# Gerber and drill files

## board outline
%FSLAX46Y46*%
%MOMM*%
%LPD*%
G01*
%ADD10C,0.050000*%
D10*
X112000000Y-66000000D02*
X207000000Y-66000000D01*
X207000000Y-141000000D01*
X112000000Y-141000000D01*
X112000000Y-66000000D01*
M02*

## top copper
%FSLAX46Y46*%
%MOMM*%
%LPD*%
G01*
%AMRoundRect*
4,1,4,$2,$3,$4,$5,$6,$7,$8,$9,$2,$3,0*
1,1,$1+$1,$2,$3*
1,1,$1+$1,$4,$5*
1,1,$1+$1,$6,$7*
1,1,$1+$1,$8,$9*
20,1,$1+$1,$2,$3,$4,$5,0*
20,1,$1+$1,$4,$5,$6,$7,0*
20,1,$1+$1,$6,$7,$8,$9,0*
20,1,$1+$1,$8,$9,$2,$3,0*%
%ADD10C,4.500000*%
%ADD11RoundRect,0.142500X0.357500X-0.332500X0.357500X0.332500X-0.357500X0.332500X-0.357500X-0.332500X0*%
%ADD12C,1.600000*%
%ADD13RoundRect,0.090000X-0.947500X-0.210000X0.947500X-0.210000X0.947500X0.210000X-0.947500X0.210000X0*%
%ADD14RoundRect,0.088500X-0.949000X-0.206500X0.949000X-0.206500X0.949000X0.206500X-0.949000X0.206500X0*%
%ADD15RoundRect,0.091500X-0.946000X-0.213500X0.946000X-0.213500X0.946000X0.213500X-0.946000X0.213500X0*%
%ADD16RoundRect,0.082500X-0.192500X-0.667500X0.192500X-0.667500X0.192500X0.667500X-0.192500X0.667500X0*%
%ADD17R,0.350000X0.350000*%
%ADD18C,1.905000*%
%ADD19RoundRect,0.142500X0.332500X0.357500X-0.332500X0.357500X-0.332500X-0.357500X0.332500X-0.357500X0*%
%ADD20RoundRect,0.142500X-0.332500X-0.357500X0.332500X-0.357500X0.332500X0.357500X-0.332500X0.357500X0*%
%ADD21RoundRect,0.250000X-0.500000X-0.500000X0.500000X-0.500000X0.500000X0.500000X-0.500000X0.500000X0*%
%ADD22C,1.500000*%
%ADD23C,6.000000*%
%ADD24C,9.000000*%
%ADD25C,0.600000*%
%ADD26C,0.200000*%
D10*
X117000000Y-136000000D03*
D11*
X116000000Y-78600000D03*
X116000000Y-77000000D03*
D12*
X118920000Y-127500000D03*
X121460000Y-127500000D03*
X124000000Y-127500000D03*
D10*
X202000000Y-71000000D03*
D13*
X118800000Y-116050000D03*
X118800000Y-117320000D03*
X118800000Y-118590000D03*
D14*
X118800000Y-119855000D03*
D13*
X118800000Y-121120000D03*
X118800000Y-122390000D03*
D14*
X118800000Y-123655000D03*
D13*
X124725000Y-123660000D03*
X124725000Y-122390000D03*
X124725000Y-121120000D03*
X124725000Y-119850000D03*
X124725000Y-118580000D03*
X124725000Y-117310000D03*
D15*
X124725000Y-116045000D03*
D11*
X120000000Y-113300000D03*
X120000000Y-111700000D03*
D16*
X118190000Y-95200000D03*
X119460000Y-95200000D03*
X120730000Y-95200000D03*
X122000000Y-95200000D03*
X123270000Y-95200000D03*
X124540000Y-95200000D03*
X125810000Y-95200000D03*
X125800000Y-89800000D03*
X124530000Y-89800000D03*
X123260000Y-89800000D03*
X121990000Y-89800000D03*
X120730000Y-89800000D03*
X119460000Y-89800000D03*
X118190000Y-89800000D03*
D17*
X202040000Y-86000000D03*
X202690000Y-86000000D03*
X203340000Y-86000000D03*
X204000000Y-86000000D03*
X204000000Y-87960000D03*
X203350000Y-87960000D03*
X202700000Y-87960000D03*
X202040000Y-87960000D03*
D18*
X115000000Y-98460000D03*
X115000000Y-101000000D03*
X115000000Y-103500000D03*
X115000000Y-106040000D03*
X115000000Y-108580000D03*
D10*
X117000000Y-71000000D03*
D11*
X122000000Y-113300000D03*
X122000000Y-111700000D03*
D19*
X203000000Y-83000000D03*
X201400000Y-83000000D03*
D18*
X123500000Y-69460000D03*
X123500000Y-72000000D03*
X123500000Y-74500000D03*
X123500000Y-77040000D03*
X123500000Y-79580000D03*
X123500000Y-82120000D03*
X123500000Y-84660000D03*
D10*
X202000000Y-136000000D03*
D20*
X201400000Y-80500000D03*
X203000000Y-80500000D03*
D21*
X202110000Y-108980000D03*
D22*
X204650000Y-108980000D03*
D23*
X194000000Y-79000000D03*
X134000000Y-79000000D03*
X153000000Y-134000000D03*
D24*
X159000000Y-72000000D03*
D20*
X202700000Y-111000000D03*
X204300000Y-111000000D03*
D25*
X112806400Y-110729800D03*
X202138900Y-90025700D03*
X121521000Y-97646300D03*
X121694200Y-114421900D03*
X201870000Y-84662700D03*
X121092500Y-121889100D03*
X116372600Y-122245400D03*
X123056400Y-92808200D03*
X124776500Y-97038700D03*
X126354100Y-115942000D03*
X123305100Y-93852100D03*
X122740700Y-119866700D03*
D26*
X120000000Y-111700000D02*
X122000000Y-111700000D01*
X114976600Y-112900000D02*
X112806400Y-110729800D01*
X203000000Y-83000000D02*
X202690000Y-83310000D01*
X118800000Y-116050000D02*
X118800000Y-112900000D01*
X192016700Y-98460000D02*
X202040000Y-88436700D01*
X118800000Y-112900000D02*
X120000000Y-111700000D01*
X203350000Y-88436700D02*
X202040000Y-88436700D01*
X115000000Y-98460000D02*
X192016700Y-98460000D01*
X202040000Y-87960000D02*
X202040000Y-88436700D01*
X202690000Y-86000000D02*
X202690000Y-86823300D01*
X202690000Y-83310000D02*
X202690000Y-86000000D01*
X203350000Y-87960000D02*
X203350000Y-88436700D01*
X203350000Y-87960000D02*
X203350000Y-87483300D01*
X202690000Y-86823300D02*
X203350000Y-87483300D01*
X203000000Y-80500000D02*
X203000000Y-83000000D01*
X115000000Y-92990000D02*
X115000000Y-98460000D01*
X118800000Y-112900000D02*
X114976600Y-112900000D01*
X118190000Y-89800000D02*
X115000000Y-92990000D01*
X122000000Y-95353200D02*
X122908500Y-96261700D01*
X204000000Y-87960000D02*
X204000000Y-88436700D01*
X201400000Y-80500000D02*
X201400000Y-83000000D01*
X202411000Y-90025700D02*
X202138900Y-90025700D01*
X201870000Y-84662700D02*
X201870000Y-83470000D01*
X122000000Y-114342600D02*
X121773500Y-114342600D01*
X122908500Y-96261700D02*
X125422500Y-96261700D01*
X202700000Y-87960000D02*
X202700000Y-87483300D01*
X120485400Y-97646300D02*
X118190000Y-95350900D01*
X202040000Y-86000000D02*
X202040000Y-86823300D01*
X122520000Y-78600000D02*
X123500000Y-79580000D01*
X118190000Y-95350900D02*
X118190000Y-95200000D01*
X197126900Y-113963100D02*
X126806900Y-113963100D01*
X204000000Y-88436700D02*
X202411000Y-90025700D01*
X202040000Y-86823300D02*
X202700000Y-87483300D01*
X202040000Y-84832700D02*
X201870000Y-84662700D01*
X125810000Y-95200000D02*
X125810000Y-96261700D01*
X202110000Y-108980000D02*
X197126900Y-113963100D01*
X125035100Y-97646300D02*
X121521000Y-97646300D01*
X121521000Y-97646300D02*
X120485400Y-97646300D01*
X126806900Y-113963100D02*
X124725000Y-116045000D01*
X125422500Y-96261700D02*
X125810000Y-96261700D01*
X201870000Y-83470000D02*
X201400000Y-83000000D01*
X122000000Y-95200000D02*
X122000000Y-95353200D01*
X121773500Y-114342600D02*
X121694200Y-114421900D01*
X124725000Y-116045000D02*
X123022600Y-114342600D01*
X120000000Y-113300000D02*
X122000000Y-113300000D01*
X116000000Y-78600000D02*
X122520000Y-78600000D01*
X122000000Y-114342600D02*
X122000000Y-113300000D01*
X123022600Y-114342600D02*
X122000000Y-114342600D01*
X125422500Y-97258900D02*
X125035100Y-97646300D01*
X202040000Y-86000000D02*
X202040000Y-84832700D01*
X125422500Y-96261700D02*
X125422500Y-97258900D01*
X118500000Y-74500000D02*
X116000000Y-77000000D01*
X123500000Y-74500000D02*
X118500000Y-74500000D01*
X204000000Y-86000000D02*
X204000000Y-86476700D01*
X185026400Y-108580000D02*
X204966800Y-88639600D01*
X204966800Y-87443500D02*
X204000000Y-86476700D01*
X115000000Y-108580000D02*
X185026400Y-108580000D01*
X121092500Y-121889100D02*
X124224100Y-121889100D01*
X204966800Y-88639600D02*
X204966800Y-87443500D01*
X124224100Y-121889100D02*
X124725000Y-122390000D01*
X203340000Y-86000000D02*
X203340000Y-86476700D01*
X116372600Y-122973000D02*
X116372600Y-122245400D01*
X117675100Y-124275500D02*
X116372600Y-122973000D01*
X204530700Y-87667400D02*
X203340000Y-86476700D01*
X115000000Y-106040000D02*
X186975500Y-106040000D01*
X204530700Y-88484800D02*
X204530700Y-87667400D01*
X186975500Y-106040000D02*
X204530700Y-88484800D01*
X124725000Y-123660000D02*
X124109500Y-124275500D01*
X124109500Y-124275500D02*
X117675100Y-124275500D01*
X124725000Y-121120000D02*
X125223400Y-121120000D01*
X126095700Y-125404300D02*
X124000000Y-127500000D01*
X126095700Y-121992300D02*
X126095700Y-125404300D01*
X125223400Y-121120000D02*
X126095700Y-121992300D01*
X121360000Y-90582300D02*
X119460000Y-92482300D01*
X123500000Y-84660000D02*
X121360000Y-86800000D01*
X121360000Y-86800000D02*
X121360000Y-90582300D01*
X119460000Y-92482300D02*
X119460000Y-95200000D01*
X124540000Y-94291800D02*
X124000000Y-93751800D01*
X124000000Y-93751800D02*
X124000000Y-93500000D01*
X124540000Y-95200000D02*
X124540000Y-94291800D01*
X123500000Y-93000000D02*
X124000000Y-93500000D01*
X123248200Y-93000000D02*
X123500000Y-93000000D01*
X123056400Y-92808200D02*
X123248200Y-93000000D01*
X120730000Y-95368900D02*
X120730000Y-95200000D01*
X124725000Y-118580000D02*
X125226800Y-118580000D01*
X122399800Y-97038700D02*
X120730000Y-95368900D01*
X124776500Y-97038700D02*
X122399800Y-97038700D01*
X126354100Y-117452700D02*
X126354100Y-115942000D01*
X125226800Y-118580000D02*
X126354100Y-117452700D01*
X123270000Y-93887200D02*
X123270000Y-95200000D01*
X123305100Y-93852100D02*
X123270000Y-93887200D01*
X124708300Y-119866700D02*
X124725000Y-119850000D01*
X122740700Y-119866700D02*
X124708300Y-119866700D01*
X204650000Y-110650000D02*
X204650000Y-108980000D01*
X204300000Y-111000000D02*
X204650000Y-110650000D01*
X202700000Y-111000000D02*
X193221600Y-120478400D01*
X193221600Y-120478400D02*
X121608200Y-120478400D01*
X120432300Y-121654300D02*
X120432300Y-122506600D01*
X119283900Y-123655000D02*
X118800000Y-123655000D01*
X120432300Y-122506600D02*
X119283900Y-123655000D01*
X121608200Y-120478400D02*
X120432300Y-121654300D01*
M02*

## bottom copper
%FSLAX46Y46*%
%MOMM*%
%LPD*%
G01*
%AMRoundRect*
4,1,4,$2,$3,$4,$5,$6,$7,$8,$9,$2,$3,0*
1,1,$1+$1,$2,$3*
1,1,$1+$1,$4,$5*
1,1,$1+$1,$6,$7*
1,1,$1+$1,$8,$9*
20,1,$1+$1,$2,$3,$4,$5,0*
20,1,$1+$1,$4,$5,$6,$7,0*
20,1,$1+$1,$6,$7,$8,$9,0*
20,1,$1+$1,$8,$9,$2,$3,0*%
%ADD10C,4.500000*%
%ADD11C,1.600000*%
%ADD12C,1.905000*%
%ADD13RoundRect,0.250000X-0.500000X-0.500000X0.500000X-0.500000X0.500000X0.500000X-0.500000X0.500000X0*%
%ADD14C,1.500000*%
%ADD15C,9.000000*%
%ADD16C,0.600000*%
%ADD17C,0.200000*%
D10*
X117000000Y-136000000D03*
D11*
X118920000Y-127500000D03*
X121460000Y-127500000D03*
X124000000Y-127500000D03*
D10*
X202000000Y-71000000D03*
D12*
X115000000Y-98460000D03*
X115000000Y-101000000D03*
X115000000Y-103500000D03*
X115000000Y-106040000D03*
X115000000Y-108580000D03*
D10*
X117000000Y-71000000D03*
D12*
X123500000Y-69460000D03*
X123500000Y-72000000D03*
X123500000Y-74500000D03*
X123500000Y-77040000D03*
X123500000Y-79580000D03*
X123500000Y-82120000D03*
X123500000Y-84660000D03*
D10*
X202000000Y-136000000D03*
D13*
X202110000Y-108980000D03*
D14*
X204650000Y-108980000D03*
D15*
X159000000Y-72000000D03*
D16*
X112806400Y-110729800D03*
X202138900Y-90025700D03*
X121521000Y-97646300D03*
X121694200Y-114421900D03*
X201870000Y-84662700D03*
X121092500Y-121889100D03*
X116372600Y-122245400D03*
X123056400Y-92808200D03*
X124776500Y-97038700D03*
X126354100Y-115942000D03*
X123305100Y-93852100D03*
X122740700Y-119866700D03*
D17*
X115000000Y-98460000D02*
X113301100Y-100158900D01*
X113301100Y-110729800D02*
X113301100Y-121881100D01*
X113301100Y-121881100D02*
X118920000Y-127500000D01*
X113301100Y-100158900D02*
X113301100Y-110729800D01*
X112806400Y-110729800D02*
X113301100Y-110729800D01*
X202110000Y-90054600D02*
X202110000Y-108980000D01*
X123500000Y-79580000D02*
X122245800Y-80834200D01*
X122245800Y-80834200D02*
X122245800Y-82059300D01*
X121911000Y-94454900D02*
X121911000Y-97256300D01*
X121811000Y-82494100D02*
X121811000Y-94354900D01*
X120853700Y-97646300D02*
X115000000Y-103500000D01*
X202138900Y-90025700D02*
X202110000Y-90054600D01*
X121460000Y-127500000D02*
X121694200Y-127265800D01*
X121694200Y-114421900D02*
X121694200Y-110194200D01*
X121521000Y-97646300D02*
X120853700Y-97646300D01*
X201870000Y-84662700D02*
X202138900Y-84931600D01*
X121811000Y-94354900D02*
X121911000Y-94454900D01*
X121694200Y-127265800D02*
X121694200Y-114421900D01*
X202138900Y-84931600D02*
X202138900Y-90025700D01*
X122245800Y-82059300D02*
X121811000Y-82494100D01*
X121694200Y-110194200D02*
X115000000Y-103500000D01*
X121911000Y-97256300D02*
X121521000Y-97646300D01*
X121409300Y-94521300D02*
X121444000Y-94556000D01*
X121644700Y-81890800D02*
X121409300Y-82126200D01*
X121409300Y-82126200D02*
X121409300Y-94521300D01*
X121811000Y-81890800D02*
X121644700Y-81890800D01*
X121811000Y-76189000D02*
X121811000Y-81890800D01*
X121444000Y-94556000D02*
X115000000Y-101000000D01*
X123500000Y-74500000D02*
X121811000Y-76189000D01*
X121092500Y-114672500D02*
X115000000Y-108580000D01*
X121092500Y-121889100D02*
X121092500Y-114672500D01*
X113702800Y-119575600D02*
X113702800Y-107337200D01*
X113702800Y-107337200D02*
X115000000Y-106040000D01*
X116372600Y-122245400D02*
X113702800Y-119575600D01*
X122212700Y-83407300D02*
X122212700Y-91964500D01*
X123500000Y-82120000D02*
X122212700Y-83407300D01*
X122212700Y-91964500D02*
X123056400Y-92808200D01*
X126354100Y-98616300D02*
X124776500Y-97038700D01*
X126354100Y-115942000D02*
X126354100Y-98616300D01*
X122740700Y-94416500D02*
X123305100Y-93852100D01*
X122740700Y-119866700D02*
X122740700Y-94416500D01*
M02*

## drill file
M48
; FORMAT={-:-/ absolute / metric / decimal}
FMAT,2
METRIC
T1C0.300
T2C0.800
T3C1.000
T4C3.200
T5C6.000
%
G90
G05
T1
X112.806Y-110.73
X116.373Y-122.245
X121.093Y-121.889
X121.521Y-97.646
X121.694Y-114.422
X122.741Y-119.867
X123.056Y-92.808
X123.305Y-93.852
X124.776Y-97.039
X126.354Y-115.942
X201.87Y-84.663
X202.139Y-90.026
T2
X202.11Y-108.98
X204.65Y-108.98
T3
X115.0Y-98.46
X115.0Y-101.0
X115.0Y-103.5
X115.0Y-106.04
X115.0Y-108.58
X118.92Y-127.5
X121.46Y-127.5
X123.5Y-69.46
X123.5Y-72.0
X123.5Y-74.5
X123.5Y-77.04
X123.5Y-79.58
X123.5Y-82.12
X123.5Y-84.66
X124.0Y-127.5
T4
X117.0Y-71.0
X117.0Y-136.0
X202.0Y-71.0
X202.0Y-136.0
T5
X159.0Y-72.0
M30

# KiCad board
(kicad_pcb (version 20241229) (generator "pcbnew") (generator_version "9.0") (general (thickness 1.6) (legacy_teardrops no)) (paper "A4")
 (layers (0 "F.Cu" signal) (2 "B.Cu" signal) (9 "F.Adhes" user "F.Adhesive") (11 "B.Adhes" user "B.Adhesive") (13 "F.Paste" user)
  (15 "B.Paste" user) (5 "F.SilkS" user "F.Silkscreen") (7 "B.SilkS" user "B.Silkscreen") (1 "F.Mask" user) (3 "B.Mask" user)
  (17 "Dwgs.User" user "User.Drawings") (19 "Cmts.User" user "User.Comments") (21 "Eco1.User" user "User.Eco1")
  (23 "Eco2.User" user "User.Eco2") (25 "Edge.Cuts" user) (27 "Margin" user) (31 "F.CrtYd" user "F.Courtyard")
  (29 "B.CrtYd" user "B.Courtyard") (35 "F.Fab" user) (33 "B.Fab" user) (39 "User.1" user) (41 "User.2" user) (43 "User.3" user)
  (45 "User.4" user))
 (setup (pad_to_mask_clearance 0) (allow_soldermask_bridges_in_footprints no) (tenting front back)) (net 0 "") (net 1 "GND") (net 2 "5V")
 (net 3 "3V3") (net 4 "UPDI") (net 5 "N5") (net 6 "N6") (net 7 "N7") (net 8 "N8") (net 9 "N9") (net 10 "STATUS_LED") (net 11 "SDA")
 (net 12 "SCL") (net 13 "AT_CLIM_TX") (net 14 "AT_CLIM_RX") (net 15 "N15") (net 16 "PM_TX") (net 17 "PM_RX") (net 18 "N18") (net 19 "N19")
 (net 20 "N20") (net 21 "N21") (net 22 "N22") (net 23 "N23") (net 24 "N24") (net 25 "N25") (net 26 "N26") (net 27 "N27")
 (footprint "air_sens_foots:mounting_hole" (layer "F.Cu") (at 116.9 145.7)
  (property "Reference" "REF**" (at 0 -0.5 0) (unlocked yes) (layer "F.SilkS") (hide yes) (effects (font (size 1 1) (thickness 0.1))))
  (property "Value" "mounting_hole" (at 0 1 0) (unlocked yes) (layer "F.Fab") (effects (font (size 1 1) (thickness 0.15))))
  (pad "" thru_hole circle (at 0.1 -9.7) (size 4.5 4.5) (drill 3.2) (layers "*.Cu" "*.Mask") (remove_unused_layers no)))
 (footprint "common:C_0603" (layer "F.Cu") (at 116 77.8 90)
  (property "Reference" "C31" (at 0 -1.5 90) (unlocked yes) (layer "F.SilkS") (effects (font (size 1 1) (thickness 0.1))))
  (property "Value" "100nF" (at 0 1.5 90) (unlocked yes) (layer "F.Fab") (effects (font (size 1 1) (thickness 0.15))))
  (pad "1" smd roundrect (at -0.8 0 90) (size 0.95 1) (layers "F.Cu" "F.Mask" "F.Paste") (roundrect_rratio 0.15) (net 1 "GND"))
  (pad "2" smd roundrect (at 0.8 0 90) (size 0.95 1) (layers "F.Cu" "F.Mask" "F.Paste") (roundrect_rratio 0.15) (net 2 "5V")))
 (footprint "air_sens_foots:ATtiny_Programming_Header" (layer "F.Cu") (at 121.46 132)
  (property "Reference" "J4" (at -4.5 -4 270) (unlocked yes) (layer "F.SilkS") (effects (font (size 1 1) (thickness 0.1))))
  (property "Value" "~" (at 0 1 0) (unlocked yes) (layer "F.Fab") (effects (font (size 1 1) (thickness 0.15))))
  (pad "1" thru_hole circle (at -2.54 -4.5 90) (size 1.6 1.6) (drill 1) (layers "*.Cu" "*.Mask") (remove_unused_layers no) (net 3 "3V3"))
  (pad "2" thru_hole circle (at 0 -4.5 90) (size 1.6 1.6) (drill 1) (layers "*.Cu" "*.Mask") (remove_unused_layers no) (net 1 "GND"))
  (pad "3" thru_hole circle (at 2.54 -4.5 90) (size 1.6 1.6) (drill 1) (layers "*.Cu" "*.Mask") (remove_unused_layers no) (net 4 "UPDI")))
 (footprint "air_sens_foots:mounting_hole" (layer "F.Cu") (at 201.9 80.7)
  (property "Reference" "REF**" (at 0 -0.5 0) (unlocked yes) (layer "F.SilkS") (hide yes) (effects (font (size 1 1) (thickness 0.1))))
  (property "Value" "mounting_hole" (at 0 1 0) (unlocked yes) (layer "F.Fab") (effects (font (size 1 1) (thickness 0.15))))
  (pad "" thru_hole circle (at 0.1 -9.7) (size 4.5 4.5) (drill 3.2) (layers "*.Cu" "*.Mask") (remove_unused_layers no)))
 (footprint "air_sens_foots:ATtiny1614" (layer "F.Cu") (at 116.0625 120.85 -90)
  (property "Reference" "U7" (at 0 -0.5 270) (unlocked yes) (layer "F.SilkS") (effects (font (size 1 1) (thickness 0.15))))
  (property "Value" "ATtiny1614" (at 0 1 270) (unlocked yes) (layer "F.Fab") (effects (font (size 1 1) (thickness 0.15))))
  (pad "1" smd roundrect (at -4.8 -2.7375) (size 2.075 0.6) (layers "F.Cu" "F.Mask" "F.Paste") (roundrect_rratio 0.15) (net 3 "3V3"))
  (pad "2" smd roundrect (at -3.53 -2.7375) (size 2.075 0.6) (layers "F.Cu" "F.Mask" "F.Paste") (roundrect_rratio 0.15) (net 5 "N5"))
  (pad "3" smd roundrect (at -2.26 -2.7375) (size 2.075 0.6) (layers "F.Cu" "F.Mask" "F.Paste") (roundrect_rratio 0.15) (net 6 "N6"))
  (pad "4" smd roundrect (at -0.995 -2.7375) (size 2.075 0.59) (layers "F.Cu" "F.Mask" "F.Paste") (roundrect_rratio 0.15) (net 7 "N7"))
  (pad "5" smd roundrect (at 0.27 -2.7375) (size 2.075 0.6) (layers "F.Cu" "F.Mask" "F.Paste") (roundrect_rratio 0.15) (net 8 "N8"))
  (pad "6" smd roundrect (at 1.54 -2.7375) (size 2.075 0.6) (layers "F.Cu" "F.Mask" "F.Paste") (roundrect_rratio 0.15) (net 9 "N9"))
  (pad "7" smd roundrect (at 2.805 -2.7375) (size 2.075 0.59) (layers "F.Cu" "F.Mask" "F.Paste") (roundrect_rratio 0.15)
   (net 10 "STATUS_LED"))
  (pad "8" smd roundrect (at 2.81 -8.6625) (size 2.075 0.6) (layers "F.Cu" "F.Mask" "F.Paste") (roundrect_rratio 0.15) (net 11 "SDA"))
  (pad "9" smd roundrect (at 1.54 -8.6625) (size 2.075 0.6) (layers "F.Cu" "F.Mask" "F.Paste") (roundrect_rratio 0.15) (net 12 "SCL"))
  (pad "10" smd roundrect (at 0.27 -8.6625) (size 2.075 0.6) (layers "F.Cu" "F.Mask" "F.Paste") (roundrect_rratio 0.15) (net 4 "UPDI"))
  (pad "11" smd roundrect (at -1 -8.6625) (size 2.075 0.6) (layers "F.Cu" "F.Mask" "F.Paste") (roundrect_rratio 0.15) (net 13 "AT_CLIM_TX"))
  (pad "12" smd roundrect (at -2.27 -8.6625) (size 2.075 0.6) (layers "F.Cu" "F.Mask" "F.Paste") (roundrect_rratio 0.15)
   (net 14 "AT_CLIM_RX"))
  (pad "13" smd roundrect (at -3.54 -8.6625) (size 2.075 0.6) (layers "F.Cu" "F.Mask" "F.Paste") (roundrect_rratio 0.15) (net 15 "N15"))
  (pad "14" smd roundrect (at -4.805 -8.6625) (size 2.075 0.61) (layers "F.Cu" "F.Mask" "F.Paste") (roundrect_rratio 0.15) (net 1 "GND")))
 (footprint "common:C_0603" (layer "F.Cu") (at 120 112.5 90)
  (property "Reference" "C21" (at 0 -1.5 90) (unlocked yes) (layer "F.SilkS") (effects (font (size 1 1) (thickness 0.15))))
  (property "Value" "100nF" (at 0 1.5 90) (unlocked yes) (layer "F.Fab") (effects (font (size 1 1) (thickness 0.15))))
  (pad "1" smd roundrect (at -0.8 0 90) (size 0.95 1) (layers "F.Cu" "F.Mask" "F.Paste") (roundrect_rratio 0.15) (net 1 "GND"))
  (pad "2" smd roundrect (at 0.8 0 90) (size 0.95 1) (layers "F.Cu" "F.Mask" "F.Paste") (roundrect_rratio 0.15) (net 3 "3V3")))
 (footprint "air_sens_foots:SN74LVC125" (layer "F.Cu") (at 122 92.5)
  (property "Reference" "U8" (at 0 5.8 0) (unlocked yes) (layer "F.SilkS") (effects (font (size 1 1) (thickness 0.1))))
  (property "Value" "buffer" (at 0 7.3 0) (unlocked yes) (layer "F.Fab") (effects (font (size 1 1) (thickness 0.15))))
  (pad "1" smd roundrect (at -3.81 2.7) (size 0.55 1.5) (layers "F.Cu" "F.Mask" "F.Paste") (roundrect_rratio 0.15) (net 1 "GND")
   (clearance 0.07))
  (pad "2" smd roundrect (at -2.54 2.7) (size 0.55 1.5) (layers "F.Cu" "F.Mask" "F.Paste") (roundrect_rratio 0.15) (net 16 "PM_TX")
   (clearance 0.07))
  (pad "3" smd roundrect (at -1.27 2.7) (size 0.55 1.5) (layers "F.Cu" "F.Mask" "F.Paste") (roundrect_rratio 0.15) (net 14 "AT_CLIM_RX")
   (clearance 0.07))
  (pad "4" smd roundrect (at 0 2.7) (size 0.55 1.5) (layers "F.Cu" "F.Mask" "F.Paste") (roundrect_rratio 0.15) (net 1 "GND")
   (clearance 0.07))
  (pad "5" smd roundrect (at 1.27 2.7) (size 0.55 1.5) (layers "F.Cu" "F.Mask" "F.Paste") (roundrect_rratio 0.15) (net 13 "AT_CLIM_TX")
   (clearance 0.07))
  (pad "6" smd roundrect (at 2.54 2.7) (size 0.55 1.5) (layers "F.Cu" "F.Mask" "F.Paste") (roundrect_rratio 0.15) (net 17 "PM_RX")
   (clearance 0.07))
  (pad "7" smd roundrect (at 3.81 2.7) (size 0.55 1.5) (layers "F.Cu" "F.Mask" "F.Paste") (roundrect_rratio 0.15) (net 1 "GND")
   (clearance 0.07))
  (pad "8" smd roundrect (at 3.8 -2.7) (size 0.55 1.5) (layers "F.Cu" "F.Mask" "F.Paste") (roundrect_rratio 0.15) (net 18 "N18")
   (clearance 0.07))
  (pad "9" smd roundrect (at 2.53 -2.7) (size 0.55 1.5) (layers "F.Cu" "F.Mask" "F.Paste") (roundrect_rratio 0.15) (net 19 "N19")
   (clearance 0.07))
  (pad "10" smd roundrect (at 1.26 -2.7) (size 0.55 1.5) (layers "F.Cu" "F.Mask" "F.Paste") (roundrect_rratio 0.15) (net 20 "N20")
   (clearance 0.07))
  (pad "11" smd roundrect (at -0.01 -2.7) (size 0.55 1.5) (layers "F.Cu" "F.Mask" "F.Paste") (roundrect_rratio 0.15) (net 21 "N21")
   (clearance 0.07))
  (pad "12" smd roundrect (at -1.27 -2.7) (size 0.55 1.5) (layers "F.Cu" "F.Mask" "F.Paste") (roundrect_rratio 0.15) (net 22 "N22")
   (clearance 0.07))
  (pad "13" smd roundrect (at -2.54 -2.7) (size 0.55 1.5) (layers "F.Cu" "F.Mask" "F.Paste") (roundrect_rratio 0.15) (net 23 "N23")
   (clearance 0.07))
  (pad "14" smd roundrect (at -3.81 -2.7) (size 0.55 1.5) (layers "F.Cu" "F.Mask" "F.Paste") (roundrect_rratio 0.15) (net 3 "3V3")
   (clearance 0.07)))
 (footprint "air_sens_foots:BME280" (layer "F.Cu") (at 203.02 86.98)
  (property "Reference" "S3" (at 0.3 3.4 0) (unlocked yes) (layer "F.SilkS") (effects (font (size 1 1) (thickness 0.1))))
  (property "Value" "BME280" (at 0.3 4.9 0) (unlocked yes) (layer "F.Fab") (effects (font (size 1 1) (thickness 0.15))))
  (pad "1" smd rect (at -0.98 -0.98 90) (size 0.35 0.35) (layers "F.Cu" "F.Mask" "F.Paste") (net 1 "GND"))
  (pad "2" smd rect (at -0.33 -0.98 90) (size 0.35 0.35) (layers "F.Cu" "F.Mask" "F.Paste") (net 3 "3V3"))
  (pad "3" smd rect (at 0.32 -0.98 180) (size 0.35 0.35) (layers "F.Cu" "F.Mask" "F.Paste") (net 11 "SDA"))
  (pad "4" smd rect (at 0.98 -0.98 90) (size 0.35 0.35) (layers "F.Cu" "F.Mask" "F.Paste") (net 12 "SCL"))
  (pad "5" smd rect (at 0.98 0.98 90) (size 0.35 0.35) (layers "F.Cu" "F.Mask" "F.Paste") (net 1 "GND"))
  (pad "6" smd rect (at 0.33 0.98 90) (size 0.35 0.35) (layers "F.Cu" "F.Mask" "F.Paste") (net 3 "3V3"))
  (pad "7" smd rect (at -0.32 0.98 90) (size 0.35 0.35) (layers "F.Cu" "F.Mask" "F.Paste") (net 1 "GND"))
  (pad "8" smd rect (at -0.98 0.98 90) (size 0.35 0.35) (layers "F.Cu" "F.Mask" "F.Paste") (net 3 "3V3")))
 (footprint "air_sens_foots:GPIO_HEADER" (layer "F.Cu") (at 110.9 103.44 -90)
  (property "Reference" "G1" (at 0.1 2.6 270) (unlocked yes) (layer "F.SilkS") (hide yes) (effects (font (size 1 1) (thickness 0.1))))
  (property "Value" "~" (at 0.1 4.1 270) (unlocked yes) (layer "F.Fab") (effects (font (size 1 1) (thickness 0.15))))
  (pad "1" thru_hole circle (at -4.98 -4.1 270) (size 1.905 1.905) (drill 1) (layers "*.Cu" "*.Mask") (remove_unused_layers no)
   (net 3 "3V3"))
  (pad "2" thru_hole circle (at -2.44 -4.1 270) (size 1.905 1.905) (drill 1) (layers "*.Cu" "*.Mask") (remove_unused_layers no) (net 2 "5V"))
  (pad "3" thru_hole circle (at 0.06 -4.1 270) (size 1.905 1.905) (drill 1) (layers "*.Cu" "*.Mask") (remove_unused_layers no) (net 1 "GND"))
  (pad "4" thru_hole circle (at 2.6 -4.1 270) (size 1.905 1.905) (drill 1) (layers "*.Cu" "*.Mask") (remove_unused_layers no) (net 11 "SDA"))
  (pad "5" thru_hole circle (at 5.14 -4.1 270) (size 1.905 1.905) (drill 1) (layers "*.Cu" "*.Mask") (remove_unused_layers no)
   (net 12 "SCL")))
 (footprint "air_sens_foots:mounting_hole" (layer "F.Cu") (at 116.9 80.7)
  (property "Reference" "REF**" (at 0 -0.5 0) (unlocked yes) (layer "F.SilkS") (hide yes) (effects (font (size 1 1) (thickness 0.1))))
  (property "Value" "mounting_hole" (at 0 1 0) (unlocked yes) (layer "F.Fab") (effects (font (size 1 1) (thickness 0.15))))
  (pad "" thru_hole circle (at 0.1 -9.7) (size 4.5 4.5) (drill 3.2) (layers "*.Cu" "*.Mask") (remove_unused_layers no)))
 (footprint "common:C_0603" (layer "F.Cu") (at 122 112.5 90)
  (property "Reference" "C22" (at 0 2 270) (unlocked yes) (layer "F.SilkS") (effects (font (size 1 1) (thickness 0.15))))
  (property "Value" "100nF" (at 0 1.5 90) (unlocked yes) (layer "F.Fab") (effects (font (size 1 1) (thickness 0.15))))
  (pad "1" smd roundrect (at -0.8 0 90) (size 0.95 1) (layers "F.Cu" "F.Mask" "F.Paste") (roundrect_rratio 0.15) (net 1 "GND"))
  (pad "2" smd roundrect (at 0.8 0 90) (size 0.95 1) (layers "F.Cu" "F.Mask" "F.Paste") (roundrect_rratio 0.15) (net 3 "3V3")))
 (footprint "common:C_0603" (layer "F.Cu") (at 202.2 83 180)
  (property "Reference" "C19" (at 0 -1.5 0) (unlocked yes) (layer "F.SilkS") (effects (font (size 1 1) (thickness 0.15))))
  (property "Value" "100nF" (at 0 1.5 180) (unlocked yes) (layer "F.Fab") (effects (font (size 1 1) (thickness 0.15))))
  (pad "1" smd roundrect (at -0.8 0 180) (size 0.95 1) (layers "F.Cu" "F.Mask" "F.Paste") (roundrect_rratio 0.15) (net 3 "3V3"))
  (pad "2" smd roundrect (at 0.8 0 180) (size 0.95 1) (layers "F.Cu" "F.Mask" "F.Paste") (roundrect_rratio 0.15) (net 1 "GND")))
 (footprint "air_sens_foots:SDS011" (layer "F.Cu") (at 122.2 75.74 -90)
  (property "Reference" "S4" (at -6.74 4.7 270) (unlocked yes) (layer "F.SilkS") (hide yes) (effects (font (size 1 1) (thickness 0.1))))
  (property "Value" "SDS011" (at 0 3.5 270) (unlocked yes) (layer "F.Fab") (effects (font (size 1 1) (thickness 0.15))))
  (pad "1" thru_hole circle (at -6.28 -1.3 270) (size 1.905 1.905) (drill 1) (layers "*.Cu" "*.Mask") (remove_unused_layers no)
   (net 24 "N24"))
  (pad "2" thru_hole circle (at -3.74 -1.3 270) (size 1.905 1.905) (drill 1) (layers "*.Cu" "*.Mask") (remove_unused_layers no)
   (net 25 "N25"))
  (pad "3" thru_hole circle (at -1.24 -1.3 270) (size 1.905 1.905) (drill 1) (layers "*.Cu" "*.Mask") (remove_unused_layers no) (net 2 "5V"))
  (pad "4" thru_hole circle (at 1.3 -1.3 270) (size 1.905 1.905) (drill 1) (layers "*.Cu" "*.Mask") (remove_unused_layers no) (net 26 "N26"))
  (pad "5" thru_hole circle (at 3.84 -1.3 270) (size 1.905 1.905) (drill 1) (layers "*.Cu" "*.Mask") (remove_unused_layers no) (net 1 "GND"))
  (pad "6" thru_hole circle (at 6.38 -1.3 270) (size 1.905 1.905) (drill 1) (layers "*.Cu" "*.Mask") (remove_unused_layers no)
   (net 17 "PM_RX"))
  (pad "7" thru_hole circle (at 8.92 -1.3 270) (size 1.905 1.905) (drill 1) (layers "*.Cu" "*.Mask") (remove_unused_layers no)
   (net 16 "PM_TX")))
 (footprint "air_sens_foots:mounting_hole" (layer "F.Cu") (at 201.9 145.7)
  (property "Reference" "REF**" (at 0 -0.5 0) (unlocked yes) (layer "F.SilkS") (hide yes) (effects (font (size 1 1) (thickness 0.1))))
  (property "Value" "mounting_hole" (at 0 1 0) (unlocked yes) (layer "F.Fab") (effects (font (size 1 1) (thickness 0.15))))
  (pad "" thru_hole circle (at 0.1 -9.7) (size 4.5 4.5) (drill 3.2) (layers "*.Cu" "*.Mask") (remove_unused_layers no)))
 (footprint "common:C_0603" (layer "F.Cu") (at 202.2 80.5)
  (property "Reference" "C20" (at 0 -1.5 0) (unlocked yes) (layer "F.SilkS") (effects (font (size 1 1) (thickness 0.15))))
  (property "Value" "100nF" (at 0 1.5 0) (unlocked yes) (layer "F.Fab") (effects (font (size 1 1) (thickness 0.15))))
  (pad "1" smd roundrect (at -0.8 0) (size 0.95 1) (layers "F.Cu" "F.Mask" "F.Paste") (roundrect_rratio 0.15) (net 1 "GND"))
  (pad "2" smd roundrect (at 0.8 0) (size 0.95 1) (layers "F.Cu" "F.Mask" "F.Paste") (roundrect_rratio 0.15) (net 3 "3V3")))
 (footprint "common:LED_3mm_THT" (layer "F.Cu") (at 203.45 111.98)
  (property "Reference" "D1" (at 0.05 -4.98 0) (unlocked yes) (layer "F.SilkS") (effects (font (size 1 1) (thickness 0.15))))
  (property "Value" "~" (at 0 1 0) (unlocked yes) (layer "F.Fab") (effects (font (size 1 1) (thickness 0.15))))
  (pad "1" thru_hole roundrect (at -1.34 -3) (size 1.5 1.5) (drill 0.8) (layers "*.Cu" "*.Mask") (remove_unused_layers no)
   (roundrect_rratio 0.1666666667) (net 1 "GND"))
  (pad "2" thru_hole circle (at 1.2 -3) (size 1.5 1.5) (drill 0.8) (layers "*.Cu" "*.Mask") (remove_unused_layers no) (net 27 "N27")))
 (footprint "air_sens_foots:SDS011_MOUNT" (layer "F.Cu") (at 164 103)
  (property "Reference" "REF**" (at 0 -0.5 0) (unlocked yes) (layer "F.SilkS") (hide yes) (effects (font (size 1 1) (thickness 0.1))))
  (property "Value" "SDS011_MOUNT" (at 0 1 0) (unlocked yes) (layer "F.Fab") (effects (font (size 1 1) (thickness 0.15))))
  (pad "1" smd circle (at 30 -24) (size 6 6) (layers "F.Cu" "F.Mask" "F.Paste"))
  (pad "2" smd circle (at -30 -24) (size 6 6) (layers "F.Cu" "F.Mask" "F.Paste"))
  (pad "3" smd circle (at -11 31) (size 6 6) (layers "F.Cu" "F.Mask" "F.Paste"))
  (pad "4" thru_hole circle (at -5 -31) (size 9 9) (drill 6) (layers "*.Cu" "*.Mask") (remove_unused_layers no)))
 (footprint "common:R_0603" (layer "F.Cu") (at 203.5 111)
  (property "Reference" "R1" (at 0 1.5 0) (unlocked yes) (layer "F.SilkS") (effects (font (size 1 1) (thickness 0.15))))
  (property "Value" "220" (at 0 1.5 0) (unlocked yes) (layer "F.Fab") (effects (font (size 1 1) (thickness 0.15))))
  (pad "1" smd roundrect (at -0.8 0) (size 0.95 1) (layers "F.Cu" "F.Mask" "F.Paste") (roundrect_rratio 0.15) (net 10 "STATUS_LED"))
  (pad "2" smd roundrect (at 0.8 0) (size 0.95 1) (layers "F.Cu" "F.Mask" "F.Paste") (roundrect_rratio 0.15) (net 27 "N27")))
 (gr_rect (start 112 66) (end 207 141) (stroke (width 0.05) (type solid)) (fill no) (layer "Edge.Cuts"))
 (segment (start 120 111.7) (end 122 111.7) (width 0.2) (layer "F.Cu") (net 3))
 (segment (start 114.9766 112.9) (end 112.8064 110.7298) (width 0.2) (layer "F.Cu") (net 3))
 (segment (start 203 83) (end 202.69 83.31) (width 0.2) (layer "F.Cu") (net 3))
 (segment (start 118.8 116.05) (end 118.8 112.9) (width 0.2) (layer "F.Cu") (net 3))
 (segment (start 192.0167 98.46) (end 202.04 88.4367) (width 0.2) (layer "F.Cu") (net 3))
 (segment (start 118.8 112.9) (end 120 111.7) (width 0.2) (layer "F.Cu") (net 3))
 (segment (start 203.35 88.4367) (end 202.04 88.4367) (width 0.2) (layer "F.Cu") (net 3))
 (segment (start 115 98.46) (end 192.0167 98.46) (width 0.2) (layer "F.Cu") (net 3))
 (segment (start 202.04 87.96) (end 202.04 88.4367) (width 0.2) (layer "F.Cu") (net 3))
 (segment (start 202.69 86) (end 202.69 86.8233) (width 0.2) (layer "F.Cu") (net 3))
 (segment (start 202.69 83.31) (end 202.69 86) (width 0.2) (layer "F.Cu") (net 3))
 (segment (start 203.35 87.96) (end 203.35 88.4367) (width 0.2) (layer "F.Cu") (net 3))
 (segment (start 203.35 87.96) (end 203.35 87.4833) (width 0.2) (layer "F.Cu") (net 3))
 (segment (start 202.69 86.8233) (end 203.35 87.4833) (width 0.2) (layer "F.Cu") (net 3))
 (segment (start 203 80.5) (end 203 83) (width 0.2) (layer "F.Cu") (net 3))
 (segment (start 115 92.99) (end 115 98.46) (width 0.2) (layer "F.Cu") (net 3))
 (segment (start 118.8 112.9) (end 114.9766 112.9) (width 0.2) (layer "F.Cu") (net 3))
 (segment (start 118.19 89.8) (end 115 92.99) (width 0.2) (layer "F.Cu") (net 3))
 (via (at 112.8064 110.7298) (size 0.6) (drill 0.3) (layers "F.Cu" "B.Cu") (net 3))
 (segment (start 115 98.46) (end 113.3011 100.1589) (width 0.2) (layer "B.Cu") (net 3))
 (segment (start 113.3011 110.7298) (end 113.3011 121.8811) (width 0.2) (layer "B.Cu") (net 3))
 (segment (start 113.3011 121.8811) (end 118.92 127.5) (width 0.2) (layer "B.Cu") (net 3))
 (segment (start 113.3011 100.1589) (end 113.3011 110.7298) (width 0.2) (layer "B.Cu") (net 3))
 (segment (start 112.8064 110.7298) (end 113.3011 110.7298) (width 0.2) (layer "B.Cu") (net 3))
 (segment (start 122 95.3532) (end 122.9085 96.2617) (width 0.2) (layer "F.Cu") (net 1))
 (segment (start 204 87.96) (end 204 88.4367) (width 0.2) (layer "F.Cu") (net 1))
 (segment (start 201.4 80.5) (end 201.4 83) (width 0.2) (layer "F.Cu") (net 1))
 (segment (start 202.411 90.0257) (end 202.1389 90.0257) (width 0.2) (layer "F.Cu") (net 1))
 (segment (start 201.87 84.6627) (end 201.87 83.47) (width 0.2) (layer "F.Cu") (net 1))
 (segment (start 122 114.3426) (end 121.7735 114.3426) (width 0.2) (layer "F.Cu") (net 1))
 (segment (start 122.9085 96.2617) (end 125.4225 96.2617) (width 0.2) (layer "F.Cu") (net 1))
 (segment (start 202.7 87.96) (end 202.7 87.4833) (width 0.2) (layer "F.Cu") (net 1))
 (segment (start 120.4854 97.6463) (end 118.19 95.3509) (width 0.2) (layer "F.Cu") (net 1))
 (segment (start 202.04 86) (end 202.04 86.8233) (width 0.2) (layer "F.Cu") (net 1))
 (segment (start 122.52 78.6) (end 123.5 79.58) (width 0.2) (layer "F.Cu") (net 1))
 (segment (start 118.19 95.3509) (end 118.19 95.2) (width 0.2) (layer "F.Cu") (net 1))
 (segment (start 197.1269 113.9631) (end 126.8069 113.9631) (width 0.2) (layer "F.Cu") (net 1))
 (segment (start 204 88.4367) (end 202.411 90.0257) (width 0.2) (layer "F.Cu") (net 1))
 (segment (start 202.04 86.8233) (end 202.7 87.4833) (width 0.2) (layer "F.Cu") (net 1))
 (segment (start 202.04 84.8327) (end 201.87 84.6627) (width 0.2) (layer "F.Cu") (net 1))
 (segment (start 125.81 95.2) (end 125.81 96.2617) (width 0.2) (layer "F.Cu") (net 1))
 (segment (start 202.11 108.98) (end 197.1269 113.9631) (width 0.2) (layer "F.Cu") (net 1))
 (segment (start 125.0351 97.6463) (end 121.521 97.6463) (width 0.2) (layer "F.Cu") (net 1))
 (segment (start 121.521 97.6463) (end 120.4854 97.6463) (width 0.2) (layer "F.Cu") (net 1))
 (segment (start 126.8069 113.9631) (end 124.725 116.045) (width 0.2) (layer "F.Cu") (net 1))
 (segment (start 125.4225 96.2617) (end 125.81 96.2617) (width 0.2) (layer "F.Cu") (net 1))
 (segment (start 201.87 83.47) (end 201.4 83) (width 0.2) (layer "F.Cu") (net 1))
 (segment (start 122 95.2) (end 122 95.3532) (width 0.2) (layer "F.Cu") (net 1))
 (segment (start 121.7735 114.3426) (end 121.6942 114.4219) (width 0.2) (layer "F.Cu") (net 1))
 (segment (start 124.725 116.045) (end 123.0226 114.3426) (width 0.2) (layer "F.Cu") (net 1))
 (segment (start 120 113.3) (end 122 113.3) (width 0.2) (layer "F.Cu") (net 1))
 (segment (start 116 78.6) (end 122.52 78.6) (width 0.2) (layer "F.Cu") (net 1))
 (segment (start 122 114.3426) (end 122 113.3) (width 0.2) (layer "F.Cu") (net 1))
 (segment (start 123.0226 114.3426) (end 122 114.3426) (width 0.2) (layer "F.Cu") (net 1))
 (segment (start 125.4225 97.2589) (end 125.0351 97.6463) (width 0.2) (layer "F.Cu") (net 1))
 (segment (start 202.04 86) (end 202.04 84.8327) (width 0.2) (layer "F.Cu") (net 1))
 (segment (start 125.4225 96.2617) (end 125.4225 97.2589) (width 0.2) (layer "F.Cu") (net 1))
 (via (at 202.1389 90.0257) (size 0.6) (drill 0.3) (layers "F.Cu" "B.Cu") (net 1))
 (via (at 121.521 97.6463) (size 0.6) (drill 0.3) (layers "F.Cu" "B.Cu") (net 1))
 (via (at 121.6942 114.4219) (size 0.6) (drill 0.3) (layers "F.Cu" "B.Cu") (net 1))
 (via (at 201.87 84.6627) (size 0.6) (drill 0.3) (layers "F.Cu" "B.Cu") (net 1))
 (segment (start 202.11 90.0546) (end 202.11 108.98) (width 0.2) (layer "B.Cu") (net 1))
 (segment (start 123.5 79.58) (end 122.2458 80.8342) (width 0.2) (layer "B.Cu") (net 1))
 (segment (start 122.2458 80.8342) (end 122.2458 82.0593) (width 0.2) (layer "B.Cu") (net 1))
 (segment (start 121.911 94.4549) (end 121.911 97.2563) (width 0.2) (layer "B.Cu") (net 1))
 (segment (start 121.811 82.4941) (end 121.811 94.3549) (width 0.2) (layer "B.Cu") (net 1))
 (segment (start 120.8537 97.6463) (end 115 103.5) (width 0.2) (layer "B.Cu") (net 1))
 (segment (start 202.1389 90.0257) (end 202.11 90.0546) (width 0.2) (layer "B.Cu") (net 1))
 (segment (start 121.46 127.5) (end 121.6942 127.2658) (width 0.2) (layer "B.Cu") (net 1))
 (segment (start 121.6942 114.4219) (end 121.6942 110.1942) (width 0.2) (layer "B.Cu") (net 1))
 (segment (start 121.521 97.6463) (end 120.8537 97.6463) (width 0.2) (layer "B.Cu") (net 1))
 (segment (start 201.87 84.6627) (end 202.1389 84.9316) (width 0.2) (layer "B.Cu") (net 1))
 (segment (start 121.811 94.3549) (end 121.911 94.4549) (width 0.2) (layer "B.Cu") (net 1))
 (segment (start 121.6942 127.2658) (end 121.6942 114.4219) (width 0.2) (layer "B.Cu") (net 1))
 (segment (start 202.1389 84.9316) (end 202.1389 90.0257) (width 0.2) (layer "B.Cu") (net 1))
 (segment (start 122.2458 82.0593) (end 121.811 82.4941) (width 0.2) (layer "B.Cu") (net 1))
 (segment (start 121.6942 110.1942) (end 115 103.5) (width 0.2) (layer "B.Cu") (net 1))
 (segment (start 121.911 97.2563) (end 121.521 97.6463) (width 0.2) (layer "B.Cu") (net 1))
 (segment (start 118.5 74.5) (end 116 77) (width 0.2) (layer "F.Cu") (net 2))
 (segment (start 123.5 74.5) (end 118.5 74.5) (width 0.2) (layer "F.Cu") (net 2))
 (segment (start 121.4093 94.5213) (end 121.444 94.556) (width 0.2) (layer "B.Cu") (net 2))
 (segment (start 121.6447 81.8908) (end 121.4093 82.1262) (width 0.2) (layer "B.Cu") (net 2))
 (segment (start 121.4093 82.1262) (end 121.4093 94.5213) (width 0.2) (layer "B.Cu") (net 2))
 (segment (start 121.811 81.8908) (end 121.6447 81.8908) (width 0.2) (layer "B.Cu") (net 2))
 (segment (start 121.811 76.189) (end 121.811 81.8908) (width 0.2) (layer "B.Cu") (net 2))
 (segment (start 121.444 94.556) (end 115 101) (width 0.2) (layer "B.Cu") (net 2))
 (segment (start 123.5 74.5) (end 121.811 76.189) (width 0.2) (layer "B.Cu") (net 2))
 (segment (start 204 86) (end 204 86.4767) (width 0.2) (layer "F.Cu") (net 12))
 (segment (start 185.0264 108.58) (end 204.9668 88.6396) (width 0.2) (layer "F.Cu") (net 12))
 (segment (start 204.9668 87.4435) (end 204 86.4767) (width 0.2) (layer "F.Cu") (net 12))
 (segment (start 115 108.58) (end 185.0264 108.58) (width 0.2) (layer "F.Cu") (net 12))
 (segment (start 121.0925 121.8891) (end 124.2241 121.8891) (width 0.2) (layer "F.Cu") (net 12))
 (segment (start 204.9668 88.6396) (end 204.9668 87.4435) (width 0.2) (layer "F.Cu") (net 12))
 (segment (start 124.2241 121.8891) (end 124.725 122.39) (width 0.2) (layer "F.Cu") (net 12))
 (via (at 121.0925 121.8891) (size 0.6) (drill 0.3) (layers "F.Cu" "B.Cu") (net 12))
 (segment (start 121.0925 114.6725) (end 115 108.58) (width 0.2) (layer "B.Cu") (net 12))
 (segment (start 121.0925 121.8891) (end 121.0925 114.6725) (width 0.2) (layer "B.Cu") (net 12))
 (segment (start 203.34 86) (end 203.34 86.4767) (width 0.2) (layer "F.Cu") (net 11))
 (segment (start 116.3726 122.973) (end 116.3726 122.2454) (width 0.2) (layer "F.Cu") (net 11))
 (segment (start 117.6751 124.2755) (end 116.3726 122.973) (width 0.2) (layer "F.Cu") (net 11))
 (segment (start 204.5307 87.6674) (end 203.34 86.4767) (width 0.2) (layer "F.Cu") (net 11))
 (segment (start 115 106.04) (end 186.9755 106.04) (width 0.2) (layer "F.Cu") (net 11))
 (segment (start 204.5307 88.4848) (end 204.5307 87.6674) (width 0.2) (layer "F.Cu") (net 11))
 (segment (start 186.9755 106.04) (end 204.5307 88.4848) (width 0.2) (layer "F.Cu") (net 11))
 (segment (start 124.725 123.66) (end 124.1095 124.2755) (width 0.2) (layer "F.Cu") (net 11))
 (segment (start 124.1095 124.2755) (end 117.6751 124.2755) (width 0.2) (layer "F.Cu") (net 11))
 (via (at 116.3726 122.2454) (size 0.6) (drill 0.3) (layers "F.Cu" "B.Cu") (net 11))
 (segment (start 113.7028 119.5756) (end 113.7028 107.3372) (width 0.2) (layer "B.Cu") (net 11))
 (segment (start 113.7028 107.3372) (end 115 106.04) (width 0.2) (layer "B.Cu") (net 11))
 (segment (start 116.3726 122.2454) (end 113.7028 119.5756) (width 0.2) (layer "B.Cu") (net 11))
 (segment (start 124.725 121.12) (end 125.2234 121.12) (width 0.2) (layer "F.Cu") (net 4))
 (segment (start 126.0957 125.4043) (end 124 127.5) (width 0.2) (layer "F.Cu") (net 4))
 (segment (start 126.0957 121.9923) (end 126.0957 125.4043) (width 0.2) (layer "F.Cu") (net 4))
 (segment (start 125.2234 121.12) (end 126.0957 121.9923) (width 0.2) (layer "F.Cu") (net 4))
 (segment (start 121.36 90.5823) (end 119.46 92.4823) (width 0.2) (layer "F.Cu") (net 16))
 (segment (start 123.5 84.66) (end 121.36 86.8) (width 0.2) (layer "F.Cu") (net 16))
 (segment (start 121.36 86.8) (end 121.36 90.5823) (width 0.2) (layer "F.Cu") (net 16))
 (segment (start 119.46 92.4823) (end 119.46 95.2) (width 0.2) (layer "F.Cu") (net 16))
 (segment (start 124.54 94.2918) (end 124 93.7518) (width 0.2) (layer "F.Cu") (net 17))
 (segment (start 124 93.7518) (end 124 93.5) (width 0.2) (layer "F.Cu") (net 17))
 (segment (start 124.54 95.2) (end 124.54 94.2918) (width 0.2) (layer "F.Cu") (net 17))
 (segment (start 123.5 93) (end 124 93.5) (width 0.2) (layer "F.Cu") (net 17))
 (segment (start 123.2482 93) (end 123.5 93) (width 0.2) (layer "F.Cu") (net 17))
 (segment (start 123.0564 92.8082) (end 123.2482 93) (width 0.2) (layer "F.Cu") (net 17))
 (via (at 123.0564 92.8082) (size 0.6) (drill 0.3) (layers "F.Cu" "B.Cu") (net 17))
 (segment (start 122.2127 83.4073) (end 122.2127 91.9645) (width 0.2) (layer "B.Cu") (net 17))
 (segment (start 123.5 82.12) (end 122.2127 83.4073) (width 0.2) (layer "B.Cu") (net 17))
 (segment (start 122.2127 91.9645) (end 123.0564 92.8082) (width 0.2) (layer "B.Cu") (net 17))
 (segment (start 120.73 95.3689) (end 120.73 95.2) (width 0.2) (layer "F.Cu") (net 14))
 (segment (start 124.725 118.58) (end 125.2268 118.58) (width 0.2) (layer "F.Cu") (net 14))
 (segment (start 122.3998 97.0387) (end 120.73 95.3689) (width 0.2) (layer "F.Cu") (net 14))
 (segment (start 124.7765 97.0387) (end 122.3998 97.0387) (width 0.2) (layer "F.Cu") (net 14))
 (segment (start 126.3541 117.4527) (end 126.3541 115.942) (width 0.2) (layer "F.Cu") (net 14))
 (segment (start 125.2268 118.58) (end 126.3541 117.4527) (width 0.2) (layer "F.Cu") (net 14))
 (via (at 124.7765 97.0387) (size 0.6) (drill 0.3) (layers "F.Cu" "B.Cu") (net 14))
 (via (at 126.3541 115.942) (size 0.6) (drill 0.3) (layers "F.Cu" "B.Cu") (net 14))
 (segment (start 126.3541 98.6163) (end 124.7765 97.0387) (width 0.2) (layer "B.Cu") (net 14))
 (segment (start 126.3541 115.942) (end 126.3541 98.6163) (width 0.2) (layer "B.Cu") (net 14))
 (segment (start 123.27 93.8872) (end 123.27 95.2) (width 0.2) (layer "F.Cu") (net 13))
 (segment (start 123.3051 93.8521) (end 123.27 93.8872) (width 0.2) (layer "F.Cu") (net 13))
 (segment (start 124.7083 119.8667) (end 124.725 119.85) (width 0.2) (layer "F.Cu") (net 13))
 (segment (start 122.7407 119.8667) (end 124.7083 119.8667) (width 0.2) (layer "F.Cu") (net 13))
 (via (at 123.3051 93.8521) (size 0.6) (drill 0.3) (layers "F.Cu" "B.Cu") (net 13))
 (via (at 122.7407 119.8667) (size 0.6) (drill 0.3) (layers "F.Cu" "B.Cu") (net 13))
 (segment (start 122.7407 94.4165) (end 123.3051 93.8521) (width 0.2) (layer "B.Cu") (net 13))
 (segment (start 122.7407 119.8667) (end 122.7407 94.4165) (width 0.2) (layer "B.Cu") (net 13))
 (segment (start 204.65 110.65) (end 204.65 108.98) (width 0.2) (layer "F.Cu") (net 27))
 (segment (start 204.3 111) (end 204.65 110.65) (width 0.2) (layer "F.Cu") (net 27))
 (segment (start 202.7 111) (end 193.2216 120.4784) (width 0.2) (layer "F.Cu") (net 10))
 (segment (start 193.2216 120.4784) (end 121.6082 120.4784) (width 0.2) (layer "F.Cu") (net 10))
 (segment (start 120.4323 121.6543) (end 120.4323 122.5066) (width 0.2) (layer "F.Cu") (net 10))
 (segment (start 119.2839 123.655) (end 118.8 123.655) (width 0.2) (layer "F.Cu") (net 10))
 (segment (start 120.4323 122.5066) (end 119.2839 123.655) (width 0.2) (layer "F.Cu") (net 10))
 (segment (start 121.6082 120.4784) (end 120.4323 121.6543) (width 0.2) (layer "F.Cu") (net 10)))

